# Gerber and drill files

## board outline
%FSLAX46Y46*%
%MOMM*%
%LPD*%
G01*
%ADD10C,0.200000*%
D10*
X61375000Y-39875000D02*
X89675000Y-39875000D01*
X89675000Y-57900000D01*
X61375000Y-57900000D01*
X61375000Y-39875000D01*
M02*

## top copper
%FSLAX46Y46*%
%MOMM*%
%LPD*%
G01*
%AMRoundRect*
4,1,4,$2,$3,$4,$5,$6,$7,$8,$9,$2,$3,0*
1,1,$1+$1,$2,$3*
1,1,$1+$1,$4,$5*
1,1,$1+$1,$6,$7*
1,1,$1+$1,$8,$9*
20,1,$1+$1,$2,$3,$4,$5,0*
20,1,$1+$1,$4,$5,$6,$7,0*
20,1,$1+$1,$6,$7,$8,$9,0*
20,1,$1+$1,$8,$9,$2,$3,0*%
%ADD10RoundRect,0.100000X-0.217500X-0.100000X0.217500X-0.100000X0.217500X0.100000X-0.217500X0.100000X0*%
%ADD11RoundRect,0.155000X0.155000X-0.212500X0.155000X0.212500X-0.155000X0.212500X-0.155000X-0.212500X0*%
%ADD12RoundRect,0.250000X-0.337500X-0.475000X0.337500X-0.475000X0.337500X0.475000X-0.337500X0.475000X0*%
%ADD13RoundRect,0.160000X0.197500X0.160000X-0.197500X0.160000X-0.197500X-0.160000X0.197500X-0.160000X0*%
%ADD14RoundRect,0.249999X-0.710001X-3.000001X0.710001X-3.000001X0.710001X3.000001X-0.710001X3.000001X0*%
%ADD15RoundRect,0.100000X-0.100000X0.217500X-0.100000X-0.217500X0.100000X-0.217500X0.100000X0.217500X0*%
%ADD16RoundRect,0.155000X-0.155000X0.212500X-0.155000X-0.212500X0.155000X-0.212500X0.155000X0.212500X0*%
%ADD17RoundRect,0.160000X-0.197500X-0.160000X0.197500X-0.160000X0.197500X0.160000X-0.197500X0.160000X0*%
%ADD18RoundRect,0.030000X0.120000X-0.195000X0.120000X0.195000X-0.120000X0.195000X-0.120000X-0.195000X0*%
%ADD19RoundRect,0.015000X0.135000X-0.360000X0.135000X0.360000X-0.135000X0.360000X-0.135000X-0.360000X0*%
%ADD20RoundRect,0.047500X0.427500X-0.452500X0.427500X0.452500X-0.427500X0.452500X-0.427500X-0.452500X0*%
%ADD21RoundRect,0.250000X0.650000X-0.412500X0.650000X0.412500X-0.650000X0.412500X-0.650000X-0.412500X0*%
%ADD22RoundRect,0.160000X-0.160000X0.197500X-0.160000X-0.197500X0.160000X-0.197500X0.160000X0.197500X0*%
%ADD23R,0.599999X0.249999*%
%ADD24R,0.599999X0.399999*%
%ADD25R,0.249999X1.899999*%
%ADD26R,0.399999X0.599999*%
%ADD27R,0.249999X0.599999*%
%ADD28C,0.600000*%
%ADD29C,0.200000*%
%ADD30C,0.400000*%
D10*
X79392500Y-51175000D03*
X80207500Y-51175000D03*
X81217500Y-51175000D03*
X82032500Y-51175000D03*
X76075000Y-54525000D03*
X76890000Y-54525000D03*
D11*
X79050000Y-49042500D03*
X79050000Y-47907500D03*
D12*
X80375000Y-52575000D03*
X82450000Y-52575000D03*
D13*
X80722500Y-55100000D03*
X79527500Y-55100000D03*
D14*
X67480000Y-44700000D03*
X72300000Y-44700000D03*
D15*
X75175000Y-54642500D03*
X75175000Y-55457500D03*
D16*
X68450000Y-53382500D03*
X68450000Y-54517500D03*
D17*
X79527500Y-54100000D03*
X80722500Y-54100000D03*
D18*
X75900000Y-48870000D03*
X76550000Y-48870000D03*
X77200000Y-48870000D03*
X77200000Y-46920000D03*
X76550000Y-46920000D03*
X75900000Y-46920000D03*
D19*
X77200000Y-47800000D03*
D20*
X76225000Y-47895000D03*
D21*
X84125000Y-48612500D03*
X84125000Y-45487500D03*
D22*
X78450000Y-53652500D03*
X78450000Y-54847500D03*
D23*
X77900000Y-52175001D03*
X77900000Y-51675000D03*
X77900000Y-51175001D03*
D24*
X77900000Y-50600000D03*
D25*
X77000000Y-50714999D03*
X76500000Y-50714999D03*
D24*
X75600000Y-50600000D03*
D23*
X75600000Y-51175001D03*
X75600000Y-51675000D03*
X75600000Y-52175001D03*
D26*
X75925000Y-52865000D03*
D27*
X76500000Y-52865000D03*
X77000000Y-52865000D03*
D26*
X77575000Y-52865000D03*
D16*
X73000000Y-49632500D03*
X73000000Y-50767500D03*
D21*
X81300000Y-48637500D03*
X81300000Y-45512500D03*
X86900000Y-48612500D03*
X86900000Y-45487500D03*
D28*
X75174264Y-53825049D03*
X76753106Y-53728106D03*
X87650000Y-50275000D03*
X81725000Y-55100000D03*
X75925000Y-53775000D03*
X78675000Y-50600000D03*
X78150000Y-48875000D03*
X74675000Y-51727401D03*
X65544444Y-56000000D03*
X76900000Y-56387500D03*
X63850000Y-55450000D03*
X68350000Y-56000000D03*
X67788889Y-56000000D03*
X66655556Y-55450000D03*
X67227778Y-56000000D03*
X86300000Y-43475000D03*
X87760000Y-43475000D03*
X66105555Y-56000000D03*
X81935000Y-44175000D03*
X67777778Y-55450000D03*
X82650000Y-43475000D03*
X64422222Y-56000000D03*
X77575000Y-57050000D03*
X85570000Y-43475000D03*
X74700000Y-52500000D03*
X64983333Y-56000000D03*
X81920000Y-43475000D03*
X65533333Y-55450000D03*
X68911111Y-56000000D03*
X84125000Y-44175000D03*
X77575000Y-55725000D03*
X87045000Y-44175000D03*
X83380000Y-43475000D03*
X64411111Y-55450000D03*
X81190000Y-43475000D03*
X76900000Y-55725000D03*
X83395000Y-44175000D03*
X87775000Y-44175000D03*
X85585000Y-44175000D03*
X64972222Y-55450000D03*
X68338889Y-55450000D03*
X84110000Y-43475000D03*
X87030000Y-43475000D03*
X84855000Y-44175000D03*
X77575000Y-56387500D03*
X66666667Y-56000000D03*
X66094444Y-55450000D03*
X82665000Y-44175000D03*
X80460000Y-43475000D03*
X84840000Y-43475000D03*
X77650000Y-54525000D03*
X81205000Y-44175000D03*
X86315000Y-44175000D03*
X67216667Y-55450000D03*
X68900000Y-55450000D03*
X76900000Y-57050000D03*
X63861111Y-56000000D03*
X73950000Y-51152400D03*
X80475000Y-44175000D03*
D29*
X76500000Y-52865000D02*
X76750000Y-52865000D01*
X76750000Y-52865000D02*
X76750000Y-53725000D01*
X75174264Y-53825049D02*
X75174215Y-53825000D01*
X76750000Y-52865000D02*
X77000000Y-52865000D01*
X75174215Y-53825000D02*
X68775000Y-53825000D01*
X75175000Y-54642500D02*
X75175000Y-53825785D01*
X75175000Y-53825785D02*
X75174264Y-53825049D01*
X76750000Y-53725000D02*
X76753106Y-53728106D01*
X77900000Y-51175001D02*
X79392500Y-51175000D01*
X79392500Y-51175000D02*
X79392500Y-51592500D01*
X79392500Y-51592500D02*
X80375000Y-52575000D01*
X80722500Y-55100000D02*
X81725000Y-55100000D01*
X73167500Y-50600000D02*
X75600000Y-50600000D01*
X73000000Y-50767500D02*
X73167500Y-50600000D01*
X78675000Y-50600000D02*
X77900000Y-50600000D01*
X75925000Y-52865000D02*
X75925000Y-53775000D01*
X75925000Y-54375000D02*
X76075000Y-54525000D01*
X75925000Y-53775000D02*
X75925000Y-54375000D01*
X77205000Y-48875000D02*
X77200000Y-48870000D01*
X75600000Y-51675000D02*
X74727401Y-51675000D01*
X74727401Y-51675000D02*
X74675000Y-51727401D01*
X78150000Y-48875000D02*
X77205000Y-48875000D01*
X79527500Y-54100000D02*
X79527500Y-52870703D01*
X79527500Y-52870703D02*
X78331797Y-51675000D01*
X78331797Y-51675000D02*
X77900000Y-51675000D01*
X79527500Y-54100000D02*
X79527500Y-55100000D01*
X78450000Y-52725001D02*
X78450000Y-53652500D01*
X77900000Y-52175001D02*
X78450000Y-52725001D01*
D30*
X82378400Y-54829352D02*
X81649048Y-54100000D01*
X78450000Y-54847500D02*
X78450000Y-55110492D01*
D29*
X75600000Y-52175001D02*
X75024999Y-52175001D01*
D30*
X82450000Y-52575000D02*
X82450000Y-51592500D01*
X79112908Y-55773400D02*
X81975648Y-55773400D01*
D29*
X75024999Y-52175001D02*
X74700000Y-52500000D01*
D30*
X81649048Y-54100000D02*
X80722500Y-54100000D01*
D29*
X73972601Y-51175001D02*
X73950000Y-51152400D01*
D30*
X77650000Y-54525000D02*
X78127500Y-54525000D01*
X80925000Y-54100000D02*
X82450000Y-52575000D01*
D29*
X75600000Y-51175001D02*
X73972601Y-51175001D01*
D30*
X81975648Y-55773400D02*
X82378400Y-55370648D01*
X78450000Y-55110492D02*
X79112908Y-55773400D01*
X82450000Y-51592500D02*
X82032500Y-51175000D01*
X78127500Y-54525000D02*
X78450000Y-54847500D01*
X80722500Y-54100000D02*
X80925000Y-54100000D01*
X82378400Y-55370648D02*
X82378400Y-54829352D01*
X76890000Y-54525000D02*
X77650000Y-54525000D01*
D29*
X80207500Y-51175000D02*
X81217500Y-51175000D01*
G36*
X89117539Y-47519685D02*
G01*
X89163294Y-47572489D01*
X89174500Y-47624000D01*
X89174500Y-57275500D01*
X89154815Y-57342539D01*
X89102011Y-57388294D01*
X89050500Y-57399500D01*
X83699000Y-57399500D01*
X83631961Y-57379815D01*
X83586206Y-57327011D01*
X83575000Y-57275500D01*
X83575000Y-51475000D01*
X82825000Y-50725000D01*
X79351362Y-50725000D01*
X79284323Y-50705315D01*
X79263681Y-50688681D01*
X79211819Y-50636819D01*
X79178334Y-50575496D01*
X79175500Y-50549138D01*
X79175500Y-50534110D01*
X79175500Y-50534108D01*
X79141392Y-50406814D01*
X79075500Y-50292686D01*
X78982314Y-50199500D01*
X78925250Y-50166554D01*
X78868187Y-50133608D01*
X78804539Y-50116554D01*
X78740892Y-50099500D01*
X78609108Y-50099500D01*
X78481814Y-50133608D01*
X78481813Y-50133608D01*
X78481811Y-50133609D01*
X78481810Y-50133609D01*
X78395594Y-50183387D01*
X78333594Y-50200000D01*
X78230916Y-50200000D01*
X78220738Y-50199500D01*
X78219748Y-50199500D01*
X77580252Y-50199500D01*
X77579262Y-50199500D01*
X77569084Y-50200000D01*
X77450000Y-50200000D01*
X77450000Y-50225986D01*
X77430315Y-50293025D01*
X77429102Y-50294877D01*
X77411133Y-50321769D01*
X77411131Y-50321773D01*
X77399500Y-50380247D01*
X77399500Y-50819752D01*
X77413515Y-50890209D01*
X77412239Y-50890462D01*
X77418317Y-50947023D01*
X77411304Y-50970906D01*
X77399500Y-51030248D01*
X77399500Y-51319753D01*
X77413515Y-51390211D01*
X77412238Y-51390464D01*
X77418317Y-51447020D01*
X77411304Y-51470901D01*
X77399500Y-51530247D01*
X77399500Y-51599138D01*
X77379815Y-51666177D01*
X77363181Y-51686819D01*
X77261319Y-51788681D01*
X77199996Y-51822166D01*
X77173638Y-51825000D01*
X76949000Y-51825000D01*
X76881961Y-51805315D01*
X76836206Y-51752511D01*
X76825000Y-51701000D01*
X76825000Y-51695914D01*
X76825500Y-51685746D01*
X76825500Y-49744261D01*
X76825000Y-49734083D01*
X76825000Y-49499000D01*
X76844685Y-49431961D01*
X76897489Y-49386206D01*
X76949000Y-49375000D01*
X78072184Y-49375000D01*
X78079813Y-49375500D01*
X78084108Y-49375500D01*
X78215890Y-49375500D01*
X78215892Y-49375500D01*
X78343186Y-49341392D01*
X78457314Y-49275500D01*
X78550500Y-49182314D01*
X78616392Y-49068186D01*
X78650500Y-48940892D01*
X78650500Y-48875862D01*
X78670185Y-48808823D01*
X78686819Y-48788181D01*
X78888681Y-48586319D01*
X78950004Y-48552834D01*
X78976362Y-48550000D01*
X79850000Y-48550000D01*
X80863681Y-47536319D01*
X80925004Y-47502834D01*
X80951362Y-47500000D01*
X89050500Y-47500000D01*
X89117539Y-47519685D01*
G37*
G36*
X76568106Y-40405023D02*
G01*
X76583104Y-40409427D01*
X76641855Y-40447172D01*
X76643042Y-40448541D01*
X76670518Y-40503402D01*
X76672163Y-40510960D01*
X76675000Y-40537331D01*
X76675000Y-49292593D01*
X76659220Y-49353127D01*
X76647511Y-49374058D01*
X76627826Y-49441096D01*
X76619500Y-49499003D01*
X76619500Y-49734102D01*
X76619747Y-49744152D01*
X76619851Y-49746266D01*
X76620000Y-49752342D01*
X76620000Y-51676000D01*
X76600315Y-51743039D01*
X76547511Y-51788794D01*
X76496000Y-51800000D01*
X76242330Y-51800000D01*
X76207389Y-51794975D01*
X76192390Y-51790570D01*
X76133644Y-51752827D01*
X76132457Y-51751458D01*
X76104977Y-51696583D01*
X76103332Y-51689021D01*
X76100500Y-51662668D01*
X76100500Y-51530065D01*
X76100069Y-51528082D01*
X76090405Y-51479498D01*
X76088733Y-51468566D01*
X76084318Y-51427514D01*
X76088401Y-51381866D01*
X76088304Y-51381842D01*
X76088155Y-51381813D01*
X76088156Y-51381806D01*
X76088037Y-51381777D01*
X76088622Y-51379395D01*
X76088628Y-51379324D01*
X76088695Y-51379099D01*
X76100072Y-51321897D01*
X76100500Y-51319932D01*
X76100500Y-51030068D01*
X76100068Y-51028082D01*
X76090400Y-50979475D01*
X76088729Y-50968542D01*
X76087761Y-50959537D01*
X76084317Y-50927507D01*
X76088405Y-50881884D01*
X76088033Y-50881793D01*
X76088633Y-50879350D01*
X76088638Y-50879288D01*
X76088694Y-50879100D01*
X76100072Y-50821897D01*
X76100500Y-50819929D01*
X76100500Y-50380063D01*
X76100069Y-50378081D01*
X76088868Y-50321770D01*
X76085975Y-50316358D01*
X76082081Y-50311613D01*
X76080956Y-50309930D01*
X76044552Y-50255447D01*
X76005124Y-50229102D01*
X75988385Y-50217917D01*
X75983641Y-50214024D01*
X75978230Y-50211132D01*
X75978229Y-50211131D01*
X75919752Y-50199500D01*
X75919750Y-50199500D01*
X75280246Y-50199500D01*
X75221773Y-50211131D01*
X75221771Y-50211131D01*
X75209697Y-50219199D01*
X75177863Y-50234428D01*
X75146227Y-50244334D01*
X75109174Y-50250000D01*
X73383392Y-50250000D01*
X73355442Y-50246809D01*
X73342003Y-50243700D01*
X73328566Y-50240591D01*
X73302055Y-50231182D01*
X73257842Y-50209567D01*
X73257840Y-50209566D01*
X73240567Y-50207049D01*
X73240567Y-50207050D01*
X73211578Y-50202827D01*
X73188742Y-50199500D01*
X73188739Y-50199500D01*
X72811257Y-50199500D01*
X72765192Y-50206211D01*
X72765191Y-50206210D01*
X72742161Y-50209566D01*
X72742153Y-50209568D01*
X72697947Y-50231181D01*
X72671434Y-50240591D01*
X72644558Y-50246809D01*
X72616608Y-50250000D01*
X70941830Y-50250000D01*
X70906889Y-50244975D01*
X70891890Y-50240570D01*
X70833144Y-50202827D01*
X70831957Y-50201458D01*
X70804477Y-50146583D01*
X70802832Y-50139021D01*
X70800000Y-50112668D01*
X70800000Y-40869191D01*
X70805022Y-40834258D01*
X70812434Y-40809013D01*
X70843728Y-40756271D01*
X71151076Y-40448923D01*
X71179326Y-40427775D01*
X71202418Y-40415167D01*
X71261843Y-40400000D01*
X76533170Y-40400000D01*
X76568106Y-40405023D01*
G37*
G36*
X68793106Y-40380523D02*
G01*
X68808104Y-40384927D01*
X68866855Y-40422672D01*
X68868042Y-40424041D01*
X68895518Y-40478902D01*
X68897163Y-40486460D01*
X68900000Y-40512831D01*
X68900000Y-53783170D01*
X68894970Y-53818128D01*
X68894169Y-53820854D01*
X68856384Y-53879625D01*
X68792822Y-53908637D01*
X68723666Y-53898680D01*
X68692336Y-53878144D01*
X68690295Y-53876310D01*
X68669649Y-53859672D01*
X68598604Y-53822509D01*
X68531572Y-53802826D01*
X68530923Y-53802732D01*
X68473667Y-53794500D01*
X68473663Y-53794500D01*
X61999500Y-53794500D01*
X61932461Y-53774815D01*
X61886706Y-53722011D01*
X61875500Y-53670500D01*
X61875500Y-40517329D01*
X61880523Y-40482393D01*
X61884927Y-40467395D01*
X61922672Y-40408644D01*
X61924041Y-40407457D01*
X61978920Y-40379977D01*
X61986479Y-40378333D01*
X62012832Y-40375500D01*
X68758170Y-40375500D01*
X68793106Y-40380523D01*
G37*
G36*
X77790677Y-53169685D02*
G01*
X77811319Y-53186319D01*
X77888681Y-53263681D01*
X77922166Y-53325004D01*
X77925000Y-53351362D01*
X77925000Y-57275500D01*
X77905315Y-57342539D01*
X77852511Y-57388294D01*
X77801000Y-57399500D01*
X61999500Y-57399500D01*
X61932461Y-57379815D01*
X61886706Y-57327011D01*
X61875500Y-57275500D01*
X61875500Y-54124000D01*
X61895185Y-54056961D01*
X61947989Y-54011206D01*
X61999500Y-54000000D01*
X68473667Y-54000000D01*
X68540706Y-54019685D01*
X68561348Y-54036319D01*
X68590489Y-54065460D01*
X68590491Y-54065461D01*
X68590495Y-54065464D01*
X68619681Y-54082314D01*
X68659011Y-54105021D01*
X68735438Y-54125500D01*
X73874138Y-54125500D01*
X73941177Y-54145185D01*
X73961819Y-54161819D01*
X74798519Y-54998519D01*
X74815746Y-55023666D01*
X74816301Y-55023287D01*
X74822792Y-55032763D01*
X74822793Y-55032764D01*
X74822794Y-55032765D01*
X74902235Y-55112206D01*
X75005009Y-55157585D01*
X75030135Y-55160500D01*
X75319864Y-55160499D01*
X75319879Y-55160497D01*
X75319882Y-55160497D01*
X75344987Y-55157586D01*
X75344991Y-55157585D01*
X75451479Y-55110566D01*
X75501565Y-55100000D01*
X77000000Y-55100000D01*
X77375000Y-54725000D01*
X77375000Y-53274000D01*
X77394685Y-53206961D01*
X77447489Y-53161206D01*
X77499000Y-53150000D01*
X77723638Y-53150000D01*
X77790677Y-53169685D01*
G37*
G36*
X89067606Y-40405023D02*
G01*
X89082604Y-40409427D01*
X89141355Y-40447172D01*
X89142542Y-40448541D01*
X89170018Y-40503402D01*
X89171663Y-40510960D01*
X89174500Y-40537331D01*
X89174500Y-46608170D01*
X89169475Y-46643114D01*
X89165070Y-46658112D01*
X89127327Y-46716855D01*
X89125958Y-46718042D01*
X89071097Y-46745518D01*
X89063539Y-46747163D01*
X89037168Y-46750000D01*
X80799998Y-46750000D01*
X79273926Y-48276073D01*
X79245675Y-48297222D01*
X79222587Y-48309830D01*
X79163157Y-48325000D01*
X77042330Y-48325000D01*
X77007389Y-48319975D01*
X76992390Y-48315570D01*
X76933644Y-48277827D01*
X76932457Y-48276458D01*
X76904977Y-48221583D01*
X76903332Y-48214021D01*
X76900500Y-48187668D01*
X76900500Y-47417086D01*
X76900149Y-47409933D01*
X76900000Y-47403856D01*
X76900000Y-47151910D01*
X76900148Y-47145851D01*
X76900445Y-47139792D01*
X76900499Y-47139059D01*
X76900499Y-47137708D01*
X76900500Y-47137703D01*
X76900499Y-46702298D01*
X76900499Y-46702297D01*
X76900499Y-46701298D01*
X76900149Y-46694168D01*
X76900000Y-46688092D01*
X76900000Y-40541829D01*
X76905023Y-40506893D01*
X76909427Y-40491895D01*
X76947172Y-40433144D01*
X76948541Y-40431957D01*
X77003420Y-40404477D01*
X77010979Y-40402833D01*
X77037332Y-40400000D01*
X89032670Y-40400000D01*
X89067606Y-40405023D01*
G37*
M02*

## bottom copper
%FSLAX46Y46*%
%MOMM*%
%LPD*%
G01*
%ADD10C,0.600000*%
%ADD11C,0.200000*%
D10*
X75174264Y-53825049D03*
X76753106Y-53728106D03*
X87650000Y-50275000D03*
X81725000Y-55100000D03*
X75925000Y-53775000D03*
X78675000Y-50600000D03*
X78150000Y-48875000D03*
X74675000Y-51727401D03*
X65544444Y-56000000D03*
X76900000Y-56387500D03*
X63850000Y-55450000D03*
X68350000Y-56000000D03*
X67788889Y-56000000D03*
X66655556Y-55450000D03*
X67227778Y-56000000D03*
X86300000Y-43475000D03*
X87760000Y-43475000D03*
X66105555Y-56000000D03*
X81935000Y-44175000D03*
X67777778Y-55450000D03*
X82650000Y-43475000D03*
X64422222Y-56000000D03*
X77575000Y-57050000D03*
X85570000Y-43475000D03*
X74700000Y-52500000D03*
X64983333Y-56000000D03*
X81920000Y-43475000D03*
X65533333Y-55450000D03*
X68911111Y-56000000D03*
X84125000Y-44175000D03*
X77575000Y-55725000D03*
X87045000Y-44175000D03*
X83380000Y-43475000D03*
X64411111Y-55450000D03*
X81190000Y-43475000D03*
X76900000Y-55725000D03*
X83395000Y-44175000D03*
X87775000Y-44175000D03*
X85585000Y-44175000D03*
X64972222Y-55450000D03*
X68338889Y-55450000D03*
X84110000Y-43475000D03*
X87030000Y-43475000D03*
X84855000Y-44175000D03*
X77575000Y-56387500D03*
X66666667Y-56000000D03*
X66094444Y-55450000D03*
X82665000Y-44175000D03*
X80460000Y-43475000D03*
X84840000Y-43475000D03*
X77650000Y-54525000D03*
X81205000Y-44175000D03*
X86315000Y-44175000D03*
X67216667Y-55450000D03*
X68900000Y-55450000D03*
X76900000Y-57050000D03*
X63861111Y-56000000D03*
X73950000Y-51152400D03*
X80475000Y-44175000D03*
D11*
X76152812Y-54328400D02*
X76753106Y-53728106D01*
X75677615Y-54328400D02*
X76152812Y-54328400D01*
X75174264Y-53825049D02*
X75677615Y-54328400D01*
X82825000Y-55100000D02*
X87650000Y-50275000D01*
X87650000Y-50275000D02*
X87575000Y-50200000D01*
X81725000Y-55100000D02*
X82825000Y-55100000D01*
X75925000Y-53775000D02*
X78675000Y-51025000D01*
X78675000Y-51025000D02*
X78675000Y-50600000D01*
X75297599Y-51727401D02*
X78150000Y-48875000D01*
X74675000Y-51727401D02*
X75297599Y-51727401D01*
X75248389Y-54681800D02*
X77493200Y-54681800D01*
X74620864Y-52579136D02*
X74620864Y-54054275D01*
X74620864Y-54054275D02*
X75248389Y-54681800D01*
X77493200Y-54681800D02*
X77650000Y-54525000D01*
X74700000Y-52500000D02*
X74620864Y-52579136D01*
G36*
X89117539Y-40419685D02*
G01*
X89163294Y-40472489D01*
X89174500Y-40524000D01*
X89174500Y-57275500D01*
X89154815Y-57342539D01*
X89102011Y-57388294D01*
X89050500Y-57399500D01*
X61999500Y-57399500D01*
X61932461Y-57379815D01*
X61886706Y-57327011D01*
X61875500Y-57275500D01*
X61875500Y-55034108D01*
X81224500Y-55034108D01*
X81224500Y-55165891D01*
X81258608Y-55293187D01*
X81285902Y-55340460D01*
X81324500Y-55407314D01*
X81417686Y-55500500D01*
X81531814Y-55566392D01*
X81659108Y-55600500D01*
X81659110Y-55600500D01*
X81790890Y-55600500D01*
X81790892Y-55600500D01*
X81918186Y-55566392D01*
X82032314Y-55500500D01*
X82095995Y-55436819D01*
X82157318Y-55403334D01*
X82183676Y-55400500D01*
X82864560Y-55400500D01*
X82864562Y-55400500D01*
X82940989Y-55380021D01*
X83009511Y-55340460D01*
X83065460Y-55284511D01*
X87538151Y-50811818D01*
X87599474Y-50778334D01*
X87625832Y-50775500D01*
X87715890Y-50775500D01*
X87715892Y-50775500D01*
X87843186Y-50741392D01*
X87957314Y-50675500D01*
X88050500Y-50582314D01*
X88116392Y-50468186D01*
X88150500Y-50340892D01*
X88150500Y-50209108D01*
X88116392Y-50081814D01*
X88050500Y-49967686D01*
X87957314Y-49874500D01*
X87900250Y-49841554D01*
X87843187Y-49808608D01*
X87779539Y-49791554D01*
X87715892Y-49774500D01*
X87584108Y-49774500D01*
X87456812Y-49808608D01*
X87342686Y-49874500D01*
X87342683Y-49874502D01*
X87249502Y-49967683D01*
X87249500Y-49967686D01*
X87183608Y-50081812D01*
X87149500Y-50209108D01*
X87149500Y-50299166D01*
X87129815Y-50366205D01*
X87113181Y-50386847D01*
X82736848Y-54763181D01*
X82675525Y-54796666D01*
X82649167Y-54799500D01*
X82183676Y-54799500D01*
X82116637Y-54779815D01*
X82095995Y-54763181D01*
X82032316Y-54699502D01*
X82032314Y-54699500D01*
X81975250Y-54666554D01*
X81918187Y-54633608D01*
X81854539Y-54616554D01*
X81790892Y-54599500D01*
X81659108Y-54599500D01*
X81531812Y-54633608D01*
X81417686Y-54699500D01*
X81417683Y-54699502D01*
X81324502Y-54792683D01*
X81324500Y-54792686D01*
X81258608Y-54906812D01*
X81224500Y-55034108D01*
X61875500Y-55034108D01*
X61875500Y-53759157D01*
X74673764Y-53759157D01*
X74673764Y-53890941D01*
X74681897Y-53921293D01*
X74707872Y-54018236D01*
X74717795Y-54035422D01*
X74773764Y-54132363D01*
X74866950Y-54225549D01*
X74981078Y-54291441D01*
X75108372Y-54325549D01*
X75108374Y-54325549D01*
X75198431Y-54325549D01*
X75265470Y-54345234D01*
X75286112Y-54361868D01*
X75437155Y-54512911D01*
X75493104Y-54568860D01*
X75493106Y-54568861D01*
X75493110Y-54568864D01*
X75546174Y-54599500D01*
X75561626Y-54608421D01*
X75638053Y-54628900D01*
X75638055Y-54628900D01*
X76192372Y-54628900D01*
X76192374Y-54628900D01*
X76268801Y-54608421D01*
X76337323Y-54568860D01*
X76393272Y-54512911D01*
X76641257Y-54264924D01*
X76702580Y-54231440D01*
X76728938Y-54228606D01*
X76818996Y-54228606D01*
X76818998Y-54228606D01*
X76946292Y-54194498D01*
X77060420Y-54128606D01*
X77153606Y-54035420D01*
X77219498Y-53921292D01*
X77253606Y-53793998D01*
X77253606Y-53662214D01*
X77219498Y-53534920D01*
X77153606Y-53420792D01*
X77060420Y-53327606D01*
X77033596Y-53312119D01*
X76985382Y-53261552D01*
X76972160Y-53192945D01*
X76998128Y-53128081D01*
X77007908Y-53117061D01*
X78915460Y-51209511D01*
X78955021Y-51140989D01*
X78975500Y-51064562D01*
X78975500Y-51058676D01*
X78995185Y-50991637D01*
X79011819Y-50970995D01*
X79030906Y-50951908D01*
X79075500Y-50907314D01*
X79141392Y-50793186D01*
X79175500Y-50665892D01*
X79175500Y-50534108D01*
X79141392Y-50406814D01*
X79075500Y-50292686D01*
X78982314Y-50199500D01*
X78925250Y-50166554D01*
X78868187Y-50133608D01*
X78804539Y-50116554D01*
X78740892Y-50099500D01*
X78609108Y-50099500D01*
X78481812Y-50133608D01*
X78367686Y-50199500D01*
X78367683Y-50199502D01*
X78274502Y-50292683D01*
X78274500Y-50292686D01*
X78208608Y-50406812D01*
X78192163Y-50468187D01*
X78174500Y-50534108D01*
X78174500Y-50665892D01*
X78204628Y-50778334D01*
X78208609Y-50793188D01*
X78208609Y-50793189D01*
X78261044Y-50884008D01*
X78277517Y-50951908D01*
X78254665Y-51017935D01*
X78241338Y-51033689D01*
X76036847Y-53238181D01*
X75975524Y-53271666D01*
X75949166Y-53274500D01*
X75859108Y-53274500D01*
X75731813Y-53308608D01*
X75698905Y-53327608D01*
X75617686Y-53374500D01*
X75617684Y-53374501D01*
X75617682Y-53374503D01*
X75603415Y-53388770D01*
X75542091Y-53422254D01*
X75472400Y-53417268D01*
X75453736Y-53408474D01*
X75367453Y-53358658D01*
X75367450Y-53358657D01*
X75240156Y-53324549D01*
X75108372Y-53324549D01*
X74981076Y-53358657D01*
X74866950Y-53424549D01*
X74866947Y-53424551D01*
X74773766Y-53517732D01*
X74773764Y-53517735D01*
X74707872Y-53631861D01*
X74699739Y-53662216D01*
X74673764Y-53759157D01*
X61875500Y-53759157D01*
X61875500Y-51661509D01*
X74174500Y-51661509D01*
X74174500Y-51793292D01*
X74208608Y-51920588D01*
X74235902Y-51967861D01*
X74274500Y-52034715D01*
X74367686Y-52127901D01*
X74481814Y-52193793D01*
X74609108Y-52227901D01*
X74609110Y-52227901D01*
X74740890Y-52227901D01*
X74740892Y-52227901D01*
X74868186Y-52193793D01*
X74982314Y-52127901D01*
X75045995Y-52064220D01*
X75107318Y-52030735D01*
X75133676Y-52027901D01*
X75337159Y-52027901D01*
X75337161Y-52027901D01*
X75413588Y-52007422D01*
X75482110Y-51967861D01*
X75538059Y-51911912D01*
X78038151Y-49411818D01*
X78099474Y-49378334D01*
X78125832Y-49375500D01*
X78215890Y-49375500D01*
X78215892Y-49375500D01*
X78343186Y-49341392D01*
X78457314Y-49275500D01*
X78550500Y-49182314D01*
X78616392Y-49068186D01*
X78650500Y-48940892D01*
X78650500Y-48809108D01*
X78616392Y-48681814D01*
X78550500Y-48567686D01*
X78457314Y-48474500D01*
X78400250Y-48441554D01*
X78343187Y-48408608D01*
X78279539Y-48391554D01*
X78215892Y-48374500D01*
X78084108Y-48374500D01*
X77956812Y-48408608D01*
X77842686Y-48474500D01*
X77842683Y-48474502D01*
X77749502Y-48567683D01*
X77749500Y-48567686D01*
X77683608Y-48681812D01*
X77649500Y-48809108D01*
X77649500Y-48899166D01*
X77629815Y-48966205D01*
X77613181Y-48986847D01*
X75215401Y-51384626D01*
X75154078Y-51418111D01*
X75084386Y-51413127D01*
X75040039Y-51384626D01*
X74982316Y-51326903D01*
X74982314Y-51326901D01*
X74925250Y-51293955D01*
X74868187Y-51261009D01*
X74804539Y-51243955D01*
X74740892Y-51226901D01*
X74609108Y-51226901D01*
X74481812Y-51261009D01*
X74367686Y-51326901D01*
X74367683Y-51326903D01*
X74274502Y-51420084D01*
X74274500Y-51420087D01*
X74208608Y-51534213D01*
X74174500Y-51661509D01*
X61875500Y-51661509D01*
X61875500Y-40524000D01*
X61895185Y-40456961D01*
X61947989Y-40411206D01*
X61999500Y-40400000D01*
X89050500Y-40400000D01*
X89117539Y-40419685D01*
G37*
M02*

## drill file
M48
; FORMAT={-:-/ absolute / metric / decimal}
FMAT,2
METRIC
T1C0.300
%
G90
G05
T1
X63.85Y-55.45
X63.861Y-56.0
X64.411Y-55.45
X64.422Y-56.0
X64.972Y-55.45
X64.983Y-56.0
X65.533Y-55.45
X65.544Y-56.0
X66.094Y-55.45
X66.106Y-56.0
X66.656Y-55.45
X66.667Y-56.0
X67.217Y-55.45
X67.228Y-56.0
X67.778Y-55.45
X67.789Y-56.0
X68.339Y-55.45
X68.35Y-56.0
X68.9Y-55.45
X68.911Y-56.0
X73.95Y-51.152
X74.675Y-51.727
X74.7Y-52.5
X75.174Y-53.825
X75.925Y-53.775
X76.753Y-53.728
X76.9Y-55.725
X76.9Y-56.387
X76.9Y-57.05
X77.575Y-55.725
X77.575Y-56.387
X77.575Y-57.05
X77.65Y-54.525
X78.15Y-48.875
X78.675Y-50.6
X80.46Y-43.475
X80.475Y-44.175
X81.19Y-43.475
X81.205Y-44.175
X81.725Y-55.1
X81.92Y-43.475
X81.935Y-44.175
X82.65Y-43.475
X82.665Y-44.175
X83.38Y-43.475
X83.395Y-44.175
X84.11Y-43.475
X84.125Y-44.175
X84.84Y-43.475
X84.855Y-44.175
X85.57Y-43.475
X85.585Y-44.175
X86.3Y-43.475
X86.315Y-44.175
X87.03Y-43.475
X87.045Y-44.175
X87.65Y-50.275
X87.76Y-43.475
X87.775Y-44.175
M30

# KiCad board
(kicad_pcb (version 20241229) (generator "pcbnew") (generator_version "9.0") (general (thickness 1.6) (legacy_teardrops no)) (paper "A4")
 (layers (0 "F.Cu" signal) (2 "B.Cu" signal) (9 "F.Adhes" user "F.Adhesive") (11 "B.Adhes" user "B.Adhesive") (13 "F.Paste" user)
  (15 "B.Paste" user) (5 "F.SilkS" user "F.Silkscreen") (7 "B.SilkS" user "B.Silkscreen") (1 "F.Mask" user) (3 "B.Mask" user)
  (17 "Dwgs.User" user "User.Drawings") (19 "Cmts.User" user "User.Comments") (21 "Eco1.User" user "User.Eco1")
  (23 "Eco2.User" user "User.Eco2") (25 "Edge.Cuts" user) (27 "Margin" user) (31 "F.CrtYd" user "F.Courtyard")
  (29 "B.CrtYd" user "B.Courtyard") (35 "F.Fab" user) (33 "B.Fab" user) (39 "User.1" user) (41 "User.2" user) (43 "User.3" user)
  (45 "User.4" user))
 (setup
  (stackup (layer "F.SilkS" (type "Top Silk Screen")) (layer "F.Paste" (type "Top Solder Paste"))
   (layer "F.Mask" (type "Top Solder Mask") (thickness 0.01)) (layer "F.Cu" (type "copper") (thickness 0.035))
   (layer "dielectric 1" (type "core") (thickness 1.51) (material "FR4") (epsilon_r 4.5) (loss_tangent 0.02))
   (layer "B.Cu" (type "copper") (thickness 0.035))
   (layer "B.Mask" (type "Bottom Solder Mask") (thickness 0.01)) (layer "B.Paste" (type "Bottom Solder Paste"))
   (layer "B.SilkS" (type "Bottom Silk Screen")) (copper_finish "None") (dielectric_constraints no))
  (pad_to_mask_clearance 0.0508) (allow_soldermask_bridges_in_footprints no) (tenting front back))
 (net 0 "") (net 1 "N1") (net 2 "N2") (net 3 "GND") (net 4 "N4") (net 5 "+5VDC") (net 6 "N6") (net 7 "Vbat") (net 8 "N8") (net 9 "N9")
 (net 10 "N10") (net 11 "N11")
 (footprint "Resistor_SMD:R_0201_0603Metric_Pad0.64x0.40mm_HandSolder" (layer "F.Cu") (at 79.8 51.175)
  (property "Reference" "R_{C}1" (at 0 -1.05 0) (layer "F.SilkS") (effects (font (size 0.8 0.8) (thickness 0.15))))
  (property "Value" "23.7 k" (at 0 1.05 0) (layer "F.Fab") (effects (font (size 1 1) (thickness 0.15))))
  (pad "" smd roundrect (at -0.4325 0) (size 0.458 0.36) (layers "F.Paste") (roundrect_rratio 0.25))
  (pad "" smd roundrect (at 0.4325 0) (size 0.458 0.36) (layers "F.Paste") (roundrect_rratio 0.25))
  (pad "1" smd roundrect (at -0.4075 0) (size 0.635 0.4) (layers "F.Cu" "F.Mask") (roundrect_rratio 0.25) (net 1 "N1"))
  (pad "2" smd roundrect (at 0.4075 0) (size 0.635 0.4) (layers "F.Cu" "F.Mask") (roundrect_rratio 0.25) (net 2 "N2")))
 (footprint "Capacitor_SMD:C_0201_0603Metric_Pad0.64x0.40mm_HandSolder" (layer "F.Cu") (at 81.625 51.175)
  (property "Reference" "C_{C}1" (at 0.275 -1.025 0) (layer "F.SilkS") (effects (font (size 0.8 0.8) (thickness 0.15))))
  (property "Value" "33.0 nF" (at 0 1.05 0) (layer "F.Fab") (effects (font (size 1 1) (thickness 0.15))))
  (pad "" smd roundrect (at -0.4325 0) (size 0.458 0.36) (layers "F.Paste") (roundrect_rratio 0.25))
  (pad "" smd roundrect (at 0.4325 0) (size 0.458 0.36) (layers "F.Paste") (roundrect_rratio 0.25))
  (pad "1" smd roundrect (at -0.4075 0) (size 0.635 0.4) (layers "F.Cu" "F.Mask") (roundrect_rratio 0.25) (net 2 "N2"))
  (pad "2" smd roundrect (at 0.4075 0) (size 0.635 0.4) (layers "F.Cu" "F.Mask") (roundrect_rratio 0.25) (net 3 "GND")))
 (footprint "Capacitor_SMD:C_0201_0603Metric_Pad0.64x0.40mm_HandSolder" (layer "F.Cu") (at 76.4825 54.525)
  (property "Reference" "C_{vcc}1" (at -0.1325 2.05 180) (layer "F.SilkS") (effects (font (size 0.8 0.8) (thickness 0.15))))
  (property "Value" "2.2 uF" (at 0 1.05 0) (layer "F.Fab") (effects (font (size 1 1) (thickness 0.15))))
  (pad "" smd roundrect (at -0.4325 0) (size 0.458 0.36) (layers "F.Paste") (roundrect_rratio 0.25))
  (pad "" smd roundrect (at 0.4325 0) (size 0.458 0.36) (layers "F.Paste") (roundrect_rratio 0.25))
  (pad "1" smd roundrect (at -0.4075 0) (size 0.635 0.4) (layers "F.Cu" "F.Mask") (roundrect_rratio 0.25) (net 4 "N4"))
  (pad "2" smd roundrect (at 0.4075 0) (size 0.635 0.4) (layers "F.Cu" "F.Mask") (roundrect_rratio 0.25) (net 3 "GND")))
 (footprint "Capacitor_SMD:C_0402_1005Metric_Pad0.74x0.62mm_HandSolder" (layer "F.Cu") (at 79.05 48.475 90)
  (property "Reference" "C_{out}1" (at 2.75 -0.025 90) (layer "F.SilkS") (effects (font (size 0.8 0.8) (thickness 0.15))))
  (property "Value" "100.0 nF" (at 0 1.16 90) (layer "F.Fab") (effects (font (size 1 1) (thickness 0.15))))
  (pad "1" smd roundrect (at -0.5675 0 90) (size 0.735 0.62) (layers "F.Cu" "F.Mask" "F.Paste") (roundrect_rratio 0.25) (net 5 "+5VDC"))
  (pad "2" smd roundrect (at 0.5675 0 90) (size 0.735 0.62) (layers "F.Cu" "F.Mask" "F.Paste") (roundrect_rratio 0.25) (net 3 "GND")))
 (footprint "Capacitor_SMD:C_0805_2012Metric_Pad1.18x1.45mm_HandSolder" (layer "F.Cu") (at 81.4125 52.575)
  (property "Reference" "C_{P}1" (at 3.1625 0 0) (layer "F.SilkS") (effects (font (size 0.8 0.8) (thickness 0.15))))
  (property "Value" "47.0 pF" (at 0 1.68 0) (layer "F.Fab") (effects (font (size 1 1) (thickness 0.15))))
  (pad "1" smd roundrect (at -1.0375 0) (size 1.175 1.45) (layers "F.Cu" "F.Mask" "F.Paste") (roundrect_rratio 0.212766) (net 1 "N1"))
  (pad "2" smd roundrect (at 1.0375 0) (size 1.175 1.45) (layers "F.Cu" "F.Mask" "F.Paste") (roundrect_rratio 0.212766) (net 3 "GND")))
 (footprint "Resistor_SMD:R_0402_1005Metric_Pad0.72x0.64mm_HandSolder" (layer "F.Cu") (at 80.125 55.1 180)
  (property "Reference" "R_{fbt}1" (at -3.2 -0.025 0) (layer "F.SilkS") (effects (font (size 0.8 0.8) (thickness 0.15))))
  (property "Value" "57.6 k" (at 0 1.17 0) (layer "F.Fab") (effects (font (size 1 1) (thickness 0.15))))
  (pad "1" smd roundrect (at -0.5975 0 180) (size 0.715 0.64) (layers "F.Cu" "F.Mask" "F.Paste") (roundrect_rratio 0.25) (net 5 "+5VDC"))
  (pad "2" smd roundrect (at 0.5975 0 180) (size 0.715 0.64) (layers "F.Cu" "F.Mask" "F.Paste") (roundrect_rratio 0.25) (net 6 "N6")))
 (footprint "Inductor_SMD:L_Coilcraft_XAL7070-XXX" (layer "F.Cu") (at 69.89 44.7)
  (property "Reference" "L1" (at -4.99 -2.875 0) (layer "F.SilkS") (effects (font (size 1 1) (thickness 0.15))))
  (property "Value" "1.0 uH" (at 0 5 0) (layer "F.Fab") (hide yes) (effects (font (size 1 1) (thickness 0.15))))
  (pad "1" smd roundrect (at -2.41 0) (size 1.92 6.5) (layers "F.Cu" "F.Mask" "F.Paste") (roundrect_rratio 0.130208) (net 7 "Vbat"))
  (pad "2" smd roundrect (at 2.41 0) (size 1.92 6.5) (layers "F.Cu" "F.Mask" "F.Paste") (roundrect_rratio 0.130208) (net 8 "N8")))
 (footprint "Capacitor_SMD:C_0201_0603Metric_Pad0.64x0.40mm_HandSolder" (layer "F.Cu") (at 75.175 55.05 -90)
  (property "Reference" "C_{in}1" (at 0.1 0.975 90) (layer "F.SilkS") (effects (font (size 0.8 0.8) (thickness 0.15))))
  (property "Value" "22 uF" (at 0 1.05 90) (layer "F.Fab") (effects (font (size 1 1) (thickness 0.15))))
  (pad "" smd roundrect (at -0.4325 0 270) (size 0.458 0.36) (layers "F.Paste") (roundrect_rratio 0.25))
  (pad "" smd roundrect (at 0.4325 0 270) (size 0.458 0.36) (layers "F.Paste") (roundrect_rratio 0.25))
  (pad "1" smd roundrect (at -0.4075 0 270) (size 0.635 0.4) (layers "F.Cu" "F.Mask") (roundrect_rratio 0.25) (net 7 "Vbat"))
  (pad "2" smd roundrect (at 0.4075 0 270) (size 0.635 0.4) (layers "F.Cu" "F.Mask") (roundrect_rratio 0.25) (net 3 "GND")))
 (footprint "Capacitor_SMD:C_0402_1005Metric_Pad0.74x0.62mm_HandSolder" (layer "F.Cu") (at 68.45 53.95 -90)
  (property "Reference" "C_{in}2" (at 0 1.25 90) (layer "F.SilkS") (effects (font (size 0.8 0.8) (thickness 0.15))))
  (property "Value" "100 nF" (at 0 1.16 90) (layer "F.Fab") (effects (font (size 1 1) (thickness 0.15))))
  (pad "1" smd roundrect (at -0.5675 0 270) (size 0.735 0.62) (layers "F.Cu" "F.Mask" "F.Paste") (roundrect_rratio 0.25) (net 7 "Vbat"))
  (pad "2" smd roundrect (at 0.5675 0 270) (size 0.735 0.62) (layers "F.Cu" "F.Mask" "F.Paste") (roundrect_rratio 0.25) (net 3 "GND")))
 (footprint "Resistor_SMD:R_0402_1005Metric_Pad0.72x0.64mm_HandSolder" (layer "F.Cu") (at 80.125 54.1)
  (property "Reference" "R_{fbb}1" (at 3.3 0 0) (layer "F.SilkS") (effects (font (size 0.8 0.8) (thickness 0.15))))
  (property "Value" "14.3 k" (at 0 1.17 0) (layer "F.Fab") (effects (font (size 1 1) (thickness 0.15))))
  (pad "1" smd roundrect (at -0.5975 0) (size 0.715 0.64) (layers "F.Cu" "F.Mask" "F.Paste") (roundrect_rratio 0.25) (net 6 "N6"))
  (pad "2" smd roundrect (at 0.5975 0) (size 0.715 0.64) (layers "F.Cu" "F.Mask" "F.Paste") (roundrect_rratio 0.25) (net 3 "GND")))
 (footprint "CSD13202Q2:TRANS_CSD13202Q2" (layer "F.Cu") (at 76.55 47.895 90)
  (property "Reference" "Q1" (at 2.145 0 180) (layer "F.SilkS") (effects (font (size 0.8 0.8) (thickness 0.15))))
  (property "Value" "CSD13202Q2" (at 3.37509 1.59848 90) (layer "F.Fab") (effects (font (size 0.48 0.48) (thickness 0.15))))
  (pad "1" smd roundrect (at -0.975 -0.65 90) (size 0.45 0.3) (layers "F.Cu" "F.Mask" "F.Paste") (roundrect_rratio 0.1) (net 8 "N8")
   (solder_mask_margin 0.102))
  (pad "2" smd roundrect (at -0.975 0 90) (size 0.45 0.3) (layers "F.Cu" "F.Mask" "F.Paste") (roundrect_rratio 0.1) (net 8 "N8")
   (solder_mask_margin 0.102))
  (pad "3" smd roundrect (at -0.975 0.65 90) (size 0.45 0.3) (layers "F.Cu" "F.Mask" "F.Paste") (roundrect_rratio 0.1) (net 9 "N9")
   (solder_mask_margin 0.102))
  (pad "4" smd roundrect (at 0.975 0.65 90) (size 0.45 0.3) (layers "F.Cu" "F.Mask" "F.Paste") (roundrect_rratio 0.1) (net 3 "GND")
   (solder_mask_margin 0.102))
  (pad "5" smd roundrect (at 0.975 0 90) (size 0.45 0.3) (layers "F.Cu" "F.Mask" "F.Paste") (roundrect_rratio 0.1) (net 8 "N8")
   (solder_mask_margin 0.102))
  (pad "6" smd roundrect (at 0.975 -0.65 90) (size 0.45 0.3) (layers "F.Cu" "F.Mask" "F.Paste") (roundrect_rratio 0.1) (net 8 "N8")
   (solder_mask_margin 0.102))
  (pad "7" smd roundrect (at 0.095 0.65 90) (size 0.75 0.3) (layers "F.Cu" "F.Mask") (roundrect_rratio 0.05) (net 3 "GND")
   (solder_mask_margin 0.102))
  (pad "8" smd roundrect (at 0 -0.325 90) (size 1 0.95) (layers "F.Cu" "F.Mask") (roundrect_rratio 0.05) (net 8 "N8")
   (solder_mask_margin 0.102)))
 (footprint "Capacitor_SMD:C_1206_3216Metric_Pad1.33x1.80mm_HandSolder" (layer "F.Cu") (at 84.125 47.05 90)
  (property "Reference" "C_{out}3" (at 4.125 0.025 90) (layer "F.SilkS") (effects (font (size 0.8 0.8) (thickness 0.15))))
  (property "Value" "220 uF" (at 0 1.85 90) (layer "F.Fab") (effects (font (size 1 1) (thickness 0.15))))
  (pad "1" smd roundrect (at -1.5625 0 90) (size 1.325 1.8) (layers "F.Cu" "F.Mask" "F.Paste") (roundrect_rratio 0.188679) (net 5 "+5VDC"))
  (pad "2" smd roundrect (at 1.5625 0 90) (size 1.325 1.8) (layers "F.Cu" "F.Mask" "F.Paste") (roundrect_rratio 0.188679) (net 3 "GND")))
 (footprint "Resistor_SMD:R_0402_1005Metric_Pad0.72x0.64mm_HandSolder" (layer "F.Cu") (at 78.45 54.25 -90)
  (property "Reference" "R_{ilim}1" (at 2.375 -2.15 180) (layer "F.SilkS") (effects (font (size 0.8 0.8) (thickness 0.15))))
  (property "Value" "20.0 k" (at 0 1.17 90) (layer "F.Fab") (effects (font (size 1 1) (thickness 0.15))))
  (pad "1" smd roundrect (at -0.5975 0 270) (size 0.715 0.64) (layers "F.Cu" "F.Mask" "F.Paste") (roundrect_rratio 0.25) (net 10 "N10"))
  (pad "2" smd roundrect (at 0.5975 0 270) (size 0.715 0.64) (layers "F.Cu" "F.Mask" "F.Paste") (roundrect_rratio 0.25) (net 3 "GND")))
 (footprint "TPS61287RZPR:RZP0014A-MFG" (layer "F.Cu") (at 76.75 51.465 180)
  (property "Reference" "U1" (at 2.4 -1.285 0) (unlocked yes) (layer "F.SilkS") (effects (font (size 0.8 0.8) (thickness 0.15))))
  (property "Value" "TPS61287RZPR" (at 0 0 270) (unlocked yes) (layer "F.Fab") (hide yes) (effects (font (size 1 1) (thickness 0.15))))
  (pad "1" smd rect (at -1.15 -0.710001 270) (size 0.249999 0.599999) (layers "F.Cu" "F.Mask" "F.Paste") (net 10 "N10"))
  (pad "2" smd rect (at -1.15 -0.21 270) (size 0.249999 0.599999) (layers "F.Cu" "F.Mask" "F.Paste") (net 6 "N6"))
  (pad "3" smd rect (at -1.15 0.289999 270) (size 0.249999 0.599999) (layers "F.Cu" "F.Mask" "F.Paste") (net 1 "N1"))
  (pad "4" smd rect (at -1.15 0.865 270) (size 0.399999 0.599999) (layers "F.Cu" "F.Mask" "F.Paste") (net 4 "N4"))
  (pad "5" smd rect (at -0.25 0.750001 180) (size 0.249999 1.899999) (layers "F.Cu" "F.Mask" "F.Paste") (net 5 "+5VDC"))
  (pad "6" smd rect (at 0.25 0.750001 180) (size 0.249999 1.899999) (layers "F.Cu" "F.Mask" "F.Paste") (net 8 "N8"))
  (pad "7" smd rect (at 1.15 0.865 270) (size 0.399999 0.599999) (layers "F.Cu" "F.Mask" "F.Paste") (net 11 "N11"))
  (pad "8" smd rect (at 1.15 0.289999 270) (size 0.249999 0.599999) (layers "F.Cu" "F.Mask" "F.Paste") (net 3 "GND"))
  (pad "9" smd rect (at 1.15 -0.21 270) (size 0.249999 0.599999) (layers "F.Cu" "F.Mask" "F.Paste") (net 9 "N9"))
  (pad "10" smd rect (at 1.15 -0.710001 270) (size 0.249999 0.599999) (layers "F.Cu" "F.Mask" "F.Paste") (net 3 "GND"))
  (pad "11" smd rect (at 0.825 -1.4 180) (size 0.399999 0.599999) (layers "F.Cu" "F.Mask" "F.Paste") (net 4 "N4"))
  (pad "12" smd rect (at 0.25 -1.4 180) (size 0.249999 0.599999) (layers "F.Cu" "F.Mask" "F.Paste") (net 7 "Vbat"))
  (pad "13" smd rect (at -0.25 -1.4 180) (size 0.249999 0.599999) (layers "F.Cu" "F.Mask" "F.Paste") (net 7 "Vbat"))
  (pad "14" smd rect (at -0.825 -1.4 180) (size 0.399999 0.599999) (layers "F.Cu" "F.Mask" "F.Paste") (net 3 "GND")))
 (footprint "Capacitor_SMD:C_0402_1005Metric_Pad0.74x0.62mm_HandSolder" (layer "F.Cu") (at 73 50.2 -90)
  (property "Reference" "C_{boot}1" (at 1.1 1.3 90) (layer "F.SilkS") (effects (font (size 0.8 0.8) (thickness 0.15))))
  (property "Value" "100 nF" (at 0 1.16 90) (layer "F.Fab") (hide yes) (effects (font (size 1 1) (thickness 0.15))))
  (pad "1" smd roundrect (at -0.5675 0 270) (size 0.735 0.62) (layers "F.Cu" "F.Mask" "F.Paste") (roundrect_rratio 0.25) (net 8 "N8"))
  (pad "2" smd roundrect (at 0.5675 0 270) (size 0.735 0.62) (layers "F.Cu" "F.Mask" "F.Paste") (roundrect_rratio 0.25) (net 11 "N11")))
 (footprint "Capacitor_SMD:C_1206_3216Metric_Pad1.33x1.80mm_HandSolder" (layer "F.Cu") (at 81.3 47.075 90)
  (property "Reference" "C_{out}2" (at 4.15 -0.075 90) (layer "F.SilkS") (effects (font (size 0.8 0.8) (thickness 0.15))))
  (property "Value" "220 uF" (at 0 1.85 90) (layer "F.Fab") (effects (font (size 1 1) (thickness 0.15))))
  (pad "1" smd roundrect (at -1.5625 0 90) (size 1.325 1.8) (layers "F.Cu" "F.Mask" "F.Paste") (roundrect_rratio 0.188679) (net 5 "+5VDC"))
  (pad "2" smd roundrect (at 1.5625 0 90) (size 1.325 1.8) (layers "F.Cu" "F.Mask" "F.Paste") (roundrect_rratio 0.188679) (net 3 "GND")))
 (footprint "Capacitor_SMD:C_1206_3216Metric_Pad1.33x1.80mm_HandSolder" (layer "F.Cu") (at 86.9 47.05 90)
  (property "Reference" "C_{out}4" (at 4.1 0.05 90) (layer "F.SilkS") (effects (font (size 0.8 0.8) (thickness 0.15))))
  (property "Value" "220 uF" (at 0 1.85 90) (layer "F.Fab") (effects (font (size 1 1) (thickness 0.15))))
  (pad "1" smd roundrect (at -1.5625 0 90) (size 1.325 1.8) (layers "F.Cu" "F.Mask" "F.Paste") (roundrect_rratio 0.188679) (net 5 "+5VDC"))
  (pad "2" smd roundrect (at 1.5625 0 90) (size 1.325 1.8) (layers "F.Cu" "F.Mask" "F.Paste") (roundrect_rratio 0.188679) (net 3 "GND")))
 (gr_rect (start 61.375 39.875) (end 89.675 57.9) (stroke (width 0.2) (type default)) (fill no) (layer "Edge.Cuts"))
 (segment (start 76.5 52.865) (end 76.75 52.865) (width 0.2) (layer "F.Cu") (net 7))
 (segment (start 76.75 52.865) (end 76.75 53.725) (width 0.2) (layer "F.Cu") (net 7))
 (segment (start 75.174264 53.825049) (end 75.174215 53.825) (width 0.2) (layer "F.Cu") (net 7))
 (segment (start 76.75 52.865) (end 77 52.865) (width 0.2) (layer "F.Cu") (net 7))
 (segment (start 75.174215 53.825) (end 68.775 53.825) (width 0.2) (layer "F.Cu") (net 7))
 (segment (start 75.175 54.6425) (end 75.175 53.825785) (width 0.2) (layer "F.Cu") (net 7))
 (segment (start 75.175 53.825785) (end 75.174264 53.825049) (width 0.2) (layer "F.Cu") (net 7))
 (segment (start 76.75 53.725) (end 76.753106 53.728106) (width 0.2) (layer "F.Cu") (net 7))
 (via (at 75.174264 53.825049) (size 0.6) (drill 0.3) (layers "F.Cu" "B.Cu") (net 7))
 (via (at 76.753106 53.728106) (size 0.6) (drill 0.3) (layers "F.Cu" "B.Cu") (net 7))
 (segment (start 76.152812 54.3284) (end 76.753106 53.728106) (width 0.2) (layer "B.Cu") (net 7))
 (segment (start 75.677615 54.3284) (end 76.152812 54.3284) (width 0.2) (layer "B.Cu") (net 7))
 (segment (start 75.174264 53.825049) (end 75.677615 54.3284) (width 0.2) (layer "B.Cu") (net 7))
 (segment (start 77.9 51.175001) (end 79.3925 51.175) (width 0.2) (layer "F.Cu") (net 1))
 (segment (start 79.3925 51.175) (end 79.3925 51.5925) (width 0.2) (layer "F.Cu") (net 1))
 (segment (start 79.3925 51.5925) (end 80.375 52.575) (width 0.2) (layer "F.Cu") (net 1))
 (segment (start 80.7225 55.1) (end 81.725 55.1) (width 0.2) (layer "F.Cu") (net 5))
 (via (at 87.65 50.275) (size 0.6) (drill 0.3) (layers "F.Cu" "B.Cu") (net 5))
 (via (at 81.725 55.1) (size 0.6) (drill 0.3) (layers "F.Cu" "B.Cu") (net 5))
 (segment (start 82.825 55.1) (end 87.65 50.275) (width 0.2) (layer "B.Cu") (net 5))
 (segment (start 87.65 50.275) (end 87.575 50.2) (width 0.2) (layer "B.Cu") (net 5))
 (segment (start 81.725 55.1) (end 82.825 55.1) (width 0.2) (layer "B.Cu") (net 5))
 (segment (start 73.1675 50.6) (end 75.6 50.6) (width 0.2) (layer "F.Cu") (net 11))
 (segment (start 73 50.7675) (end 73.1675 50.6) (width 0.2) (layer "F.Cu") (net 11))
 (segment (start 78.675 50.6) (end 77.9 50.6) (width 0.2) (layer "F.Cu") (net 4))
 (segment (start 75.925 52.865) (end 75.925 53.775) (width 0.2) (layer "F.Cu") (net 4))
 (segment (start 75.925 54.375) (end 76.075 54.525) (width 0.2) (layer "F.Cu") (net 4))
 (segment (start 75.925 53.775) (end 75.925 54.375) (width 0.2) (layer "F.Cu") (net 4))
 (via (at 75.925 53.775) (size 0.6) (drill 0.3) (layers "F.Cu" "B.Cu") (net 4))
 (via (at 78.675 50.6) (size 0.6) (drill 0.3) (layers "F.Cu" "B.Cu") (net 4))
 (segment (start 75.925 53.775) (end 78.675 51.025) (width 0.2) (layer "B.Cu") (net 4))
 (segment (start 78.675 51.025) (end 78.675 50.6) (width 0.2) (layer "B.Cu") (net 4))
 (segment (start 77.205 48.875) (end 77.2 48.87) (width 0.2) (layer "F.Cu") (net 9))
 (segment (start 75.6 51.675) (end 74.727401 51.675) (width 0.2) (layer "F.Cu") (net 9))
 (segment (start 74.727401 51.675) (end 74.675 51.727401) (width 0.2) (layer "F.Cu") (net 9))
 (segment (start 78.15 48.875) (end 77.205 48.875) (width 0.2) (layer "F.Cu") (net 9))
 (via (at 78.15 48.875) (size 0.6) (drill 0.3) (layers "F.Cu" "B.Cu") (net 9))
 (via (at 74.675 51.727401) (size 0.6) (drill 0.3) (layers "F.Cu" "B.Cu") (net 9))
 (segment (start 75.297599 51.727401) (end 78.15 48.875) (width 0.2) (layer "B.Cu") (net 9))
 (segment (start 74.675 51.727401) (end 75.297599 51.727401) (width 0.2) (layer "B.Cu") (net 9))
 (segment (start 79.5275 54.1) (end 79.5275 52.870703) (width 0.2) (layer "F.Cu") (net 6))
 (segment (start 79.5275 52.870703) (end 78.331797 51.675) (width 0.2) (layer "F.Cu") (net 6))
 (segment (start 78.331797 51.675) (end 77.9 51.675) (width 0.2) (layer "F.Cu") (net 6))
 (segment (start 79.5275 54.1) (end 79.5275 55.1) (width 0.2) (layer "F.Cu") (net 6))
 (segment (start 78.45 52.725001) (end 78.45 53.6525) (width 0.2) (layer "F.Cu") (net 10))
 (segment (start 77.9 52.175001) (end 78.45 52.725001) (width 0.2) (layer "F.Cu") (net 10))
 (segment (start 82.3784 54.829352) (end 81.649048 54.1) (width 0.4) (layer "F.Cu") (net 3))
 (segment (start 78.45 54.8475) (end 78.45 55.110492) (width 0.4) (layer "F.Cu") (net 3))
 (segment (start 75.6 52.175001) (end 75.024999 52.175001) (width 0.2) (layer "F.Cu") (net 3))
 (segment (start 82.45 52.575) (end 82.45 51.5925) (width 0.4) (layer "F.Cu") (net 3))
 (segment (start 79.112908 55.7734) (end 81.975648 55.7734) (width 0.4) (layer "F.Cu") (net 3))
 (segment (start 75.024999 52.175001) (end 74.7 52.5) (width 0.2) (layer "F.Cu") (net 3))
 (segment (start 81.649048 54.1) (end 80.7225 54.1) (width 0.4) (layer "F.Cu") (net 3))
 (segment (start 73.972601 51.175001) (end 73.95 51.1524) (width 0.2) (layer "F.Cu") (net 3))
 (segment (start 77.65 54.525) (end 78.1275 54.525) (width 0.4) (layer "F.Cu") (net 3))
 (segment (start 80.925 54.1) (end 82.45 52.575) (width 0.4) (layer "F.Cu") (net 3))
 (segment (start 75.6 51.175001) (end 73.972601 51.175001) (width 0.2) (layer "F.Cu") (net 3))
 (segment (start 81.975648 55.7734) (end 82.3784 55.370648) (width 0.4) (layer "F.Cu") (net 3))
 (segment (start 78.45 55.110492) (end 79.112908 55.7734) (width 0.4) (layer "F.Cu") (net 3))
 (segment (start 82.45 51.5925) (end 82.0325 51.175) (width 0.4) (layer "F.Cu") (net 3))
 (segment (start 78.1275 54.525) (end 78.45 54.8475) (width 0.4) (layer "F.Cu") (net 3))
 (segment (start 80.7225 54.1) (end 80.925 54.1) (width 0.4) (layer "F.Cu") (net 3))
 (segment (start 82.3784 55.370648) (end 82.3784 54.829352) (width 0.4) (layer "F.Cu") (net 3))
 (segment (start 76.89 54.525) (end 77.65 54.525) (width 0.4) (layer "F.Cu") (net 3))
 (via (at 65.544444 56) (size 0.6) (drill 0.3) (layers "F.Cu" "B.Cu") (free yes) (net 3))
 (via (at 76.9 56.3875) (size 0.6) (drill 0.3) (layers "F.Cu" "B.Cu") (free yes) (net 3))
 (via (at 63.85 55.45) (size 0.6) (drill 0.3) (layers "F.Cu" "B.Cu") (free yes) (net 3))
 (via (at 68.35 56) (size 0.6) (drill 0.3) (layers "F.Cu" "B.Cu") (free yes) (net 3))
 (via (at 67.788889 56) (size 0.6) (drill 0.3) (layers "F.Cu" "B.Cu") (free yes) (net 3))
 (via (at 66.655556 55.45) (size 0.6) (drill 0.3) (layers "F.Cu" "B.Cu") (free yes) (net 3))
 (via (at 67.227778 56) (size 0.6) (drill 0.3) (layers "F.Cu" "B.Cu") (free yes) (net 3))
 (via (at 86.3 43.475) (size 0.6) (drill 0.3) (layers "F.Cu" "B.Cu") (free yes) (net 3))
 (via (at 87.76 43.475) (size 0.6) (drill 0.3) (layers "F.Cu" "B.Cu") (free yes) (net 3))
 (via (at 66.105555 56) (size 0.6) (drill 0.3) (layers "F.Cu" "B.Cu") (free yes) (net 3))
 (via (at 81.935 44.175) (size 0.6) (drill 0.3) (layers "F.Cu" "B.Cu") (free yes) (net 3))
 (via (at 67.777778 55.45) (size 0.6) (drill 0.3) (layers "F.Cu" "B.Cu") (free yes) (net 3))
 (via (at 82.65 43.475) (size 0.6) (drill 0.3) (layers "F.Cu" "B.Cu") (free yes) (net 3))
 (via (at 64.422222 56) (size 0.6) (drill 0.3) (layers "F.Cu" "B.Cu") (free yes) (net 3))
 (via (at 77.575 57.05) (size 0.6) (drill 0.3) (layers "F.Cu" "B.Cu") (free yes) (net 3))
 (via (at 85.57 43.475) (size 0.6) (drill 0.3) (layers "F.Cu" "B.Cu") (free yes) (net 3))
 (via (at 74.7 52.5) (size 0.6) (drill 0.3) (layers "F.Cu" "B.Cu") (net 3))
 (via (at 64.983333 56) (size 0.6) (drill 0.3) (layers "F.Cu" "B.Cu") (free yes) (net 3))
 (via (at 81.92 43.475) (size 0.6) (drill 0.3) (layers "F.Cu" "B.Cu") (free yes) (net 3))
 (via (at 65.533333 55.45) (size 0.6) (drill 0.3) (layers "F.Cu" "B.Cu") (free yes) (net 3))
 (via (at 68.911111 56) (size 0.6) (drill 0.3) (layers "F.Cu" "B.Cu") (free yes) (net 3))
 (via (at 84.125 44.175) (size 0.6) (drill 0.3) (layers "F.Cu" "B.Cu") (free yes) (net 3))
 (via (at 77.575 55.725) (size 0.6) (drill 0.3) (layers "F.Cu" "B.Cu") (free yes) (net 3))
 (via (at 87.045 44.175) (size 0.6) (drill 0.3) (layers "F.Cu" "B.Cu") (free yes) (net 3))
 (via (at 83.38 43.475) (size 0.6) (drill 0.3) (layers "F.Cu" "B.Cu") (free yes) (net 3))
 (via (at 64.411111 55.45) (size 0.6) (drill 0.3) (layers "F.Cu" "B.Cu") (free yes) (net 3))
 (via (at 81.19 43.475) (size 0.6) (drill 0.3) (layers "F.Cu" "B.Cu") (free yes) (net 3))
 (via (at 76.9 55.725) (size 0.6) (drill 0.3) (layers "F.Cu" "B.Cu") (free yes) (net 3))
 (via (at 83.395 44.175) (size 0.6) (drill 0.3) (layers "F.Cu" "B.Cu") (free yes) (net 3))
 (via (at 87.775 44.175) (size 0.6) (drill 0.3) (layers "F.Cu" "B.Cu") (free yes) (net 3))
 (via (at 85.585 44.175) (size 0.6) (drill 0.3) (layers "F.Cu" "B.Cu") (free yes) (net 3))
 (via (at 64.972222 55.45) (size 0.6) (drill 0.3) (layers "F.Cu" "B.Cu") (free yes) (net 3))
 (via (at 68.338889 55.45) (size 0.6) (drill 0.3) (layers "F.Cu" "B.Cu") (free yes) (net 3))
 (via (at 84.11 43.475) (size 0.6) (drill 0.3) (layers "F.Cu" "B.Cu") (free yes) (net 3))
 (via (at 87.03 43.475) (size 0.6) (drill 0.3) (layers "F.Cu" "B.Cu") (free yes) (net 3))
 (via (at 84.855 44.175) (size 0.6) (drill 0.3) (layers "F.Cu" "B.Cu") (free yes) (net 3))
 (via (at 77.575 56.3875) (size 0.6) (drill 0.3) (layers "F.Cu" "B.Cu") (free yes) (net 3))
 (via (at 66.666667 56) (size 0.6) (drill 0.3) (layers "F.Cu" "B.Cu") (free yes) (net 3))
 (via (at 66.094444 55.45) (size 0.6) (drill 0.3) (layers "F.Cu" "B.Cu") (free yes) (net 3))
 (via (at 82.665 44.175) (size 0.6) (drill 0.3) (layers "F.Cu" "B.Cu") (free yes) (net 3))
 (via (at 80.46 43.475) (size 0.6) (drill 0.3) (layers "F.Cu" "B.Cu") (free yes) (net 3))
 (via (at 84.84 43.475) (size 0.6) (drill 0.3) (layers "F.Cu" "B.Cu") (free yes) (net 3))
 (via (at 77.65 54.525) (size 0.6) (drill 0.3) (layers "F.Cu" "B.Cu") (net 3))
 (via (at 81.205 44.175) (size 0.6) (drill 0.3) (layers "F.Cu" "B.Cu") (free yes) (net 3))
 (via (at 86.315 44.175) (size 0.6) (drill 0.3) (layers "F.Cu" "B.Cu") (free yes) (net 3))
 (via (at 67.216667 55.45) (size 0.6) (drill 0.3) (layers "F.Cu" "B.Cu") (free yes) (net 3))
 (via (at 68.9 55.45) (size 0.6) (drill 0.3) (layers "F.Cu" "B.Cu") (free yes) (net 3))
 (via (at 76.9 57.05) (size 0.6) (drill 0.3) (layers "F.Cu" "B.Cu") (free yes) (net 3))
 (via (at 63.861111 56) (size 0.6) (drill 0.3) (layers "F.Cu" "B.Cu") (free yes) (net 3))
 (via (at 73.95 51.1524) (size 0.6) (drill 0.3) (layers "F.Cu" "B.Cu") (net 3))
 (via (at 80.475 44.175) (size 0.6) (drill 0.3) (layers "F.Cu" "B.Cu") (free yes) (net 3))
 (segment (start 75.248389 54.6818) (end 77.4932 54.6818) (width 0.2) (layer "B.Cu") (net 3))
 (segment (start 74.620864 52.579136) (end 74.620864 54.054275) (width 0.2) (layer "B.Cu") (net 3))
 (segment (start 74.620864 54.054275) (end 75.248389 54.6818) (width 0.2) (layer "B.Cu") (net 3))
 (segment (start 77.4932 54.6818) (end 77.65 54.525) (width 0.2) (layer "B.Cu") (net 3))
 (segment (start 74.7 52.5) (end 74.620864 52.579136) (width 0.2) (layer "B.Cu") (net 3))
 (segment (start 80.2075 51.175) (end 81.2175 51.175) (width 0.2) (layer "F.Cu") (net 2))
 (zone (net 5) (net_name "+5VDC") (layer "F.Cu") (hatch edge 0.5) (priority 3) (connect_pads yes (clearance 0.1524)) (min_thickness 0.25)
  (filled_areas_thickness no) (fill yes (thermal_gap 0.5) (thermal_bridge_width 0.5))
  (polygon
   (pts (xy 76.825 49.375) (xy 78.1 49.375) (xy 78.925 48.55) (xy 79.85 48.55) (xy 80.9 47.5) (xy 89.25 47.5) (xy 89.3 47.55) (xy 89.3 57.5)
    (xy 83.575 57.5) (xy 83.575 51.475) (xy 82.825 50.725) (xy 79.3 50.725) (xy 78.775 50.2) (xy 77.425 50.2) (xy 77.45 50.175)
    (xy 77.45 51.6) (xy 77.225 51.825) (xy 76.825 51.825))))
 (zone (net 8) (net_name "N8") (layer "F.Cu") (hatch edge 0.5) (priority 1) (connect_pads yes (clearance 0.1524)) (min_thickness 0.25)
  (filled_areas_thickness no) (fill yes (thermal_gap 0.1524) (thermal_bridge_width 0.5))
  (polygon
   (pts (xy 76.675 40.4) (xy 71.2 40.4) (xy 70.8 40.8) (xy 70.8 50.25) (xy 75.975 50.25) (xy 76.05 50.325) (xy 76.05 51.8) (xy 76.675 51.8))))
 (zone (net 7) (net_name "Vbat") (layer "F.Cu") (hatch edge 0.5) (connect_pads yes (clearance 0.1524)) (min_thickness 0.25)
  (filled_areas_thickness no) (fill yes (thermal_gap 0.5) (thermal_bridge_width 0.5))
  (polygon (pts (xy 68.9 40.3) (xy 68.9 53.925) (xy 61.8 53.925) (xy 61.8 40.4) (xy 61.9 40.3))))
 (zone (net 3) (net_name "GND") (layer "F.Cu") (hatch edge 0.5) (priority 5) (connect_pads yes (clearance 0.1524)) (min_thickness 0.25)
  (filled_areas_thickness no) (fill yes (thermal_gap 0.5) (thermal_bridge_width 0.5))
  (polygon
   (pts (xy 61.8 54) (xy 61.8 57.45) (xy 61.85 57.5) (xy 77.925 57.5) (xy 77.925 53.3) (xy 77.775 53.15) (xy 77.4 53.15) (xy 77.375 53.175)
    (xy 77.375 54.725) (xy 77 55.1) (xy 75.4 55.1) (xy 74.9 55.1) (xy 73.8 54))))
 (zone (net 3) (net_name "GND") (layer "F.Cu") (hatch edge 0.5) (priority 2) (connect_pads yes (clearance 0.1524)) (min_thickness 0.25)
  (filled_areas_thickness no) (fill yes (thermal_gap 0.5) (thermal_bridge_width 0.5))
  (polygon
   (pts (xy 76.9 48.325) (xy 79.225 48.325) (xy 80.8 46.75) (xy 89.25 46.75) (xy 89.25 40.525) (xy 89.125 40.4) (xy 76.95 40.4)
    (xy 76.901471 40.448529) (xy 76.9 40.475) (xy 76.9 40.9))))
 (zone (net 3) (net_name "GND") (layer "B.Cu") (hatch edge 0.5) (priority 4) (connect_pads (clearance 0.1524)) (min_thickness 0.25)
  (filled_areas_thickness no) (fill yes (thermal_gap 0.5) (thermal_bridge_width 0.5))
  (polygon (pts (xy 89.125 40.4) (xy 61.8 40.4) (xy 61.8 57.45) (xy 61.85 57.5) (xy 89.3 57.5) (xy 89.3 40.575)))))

